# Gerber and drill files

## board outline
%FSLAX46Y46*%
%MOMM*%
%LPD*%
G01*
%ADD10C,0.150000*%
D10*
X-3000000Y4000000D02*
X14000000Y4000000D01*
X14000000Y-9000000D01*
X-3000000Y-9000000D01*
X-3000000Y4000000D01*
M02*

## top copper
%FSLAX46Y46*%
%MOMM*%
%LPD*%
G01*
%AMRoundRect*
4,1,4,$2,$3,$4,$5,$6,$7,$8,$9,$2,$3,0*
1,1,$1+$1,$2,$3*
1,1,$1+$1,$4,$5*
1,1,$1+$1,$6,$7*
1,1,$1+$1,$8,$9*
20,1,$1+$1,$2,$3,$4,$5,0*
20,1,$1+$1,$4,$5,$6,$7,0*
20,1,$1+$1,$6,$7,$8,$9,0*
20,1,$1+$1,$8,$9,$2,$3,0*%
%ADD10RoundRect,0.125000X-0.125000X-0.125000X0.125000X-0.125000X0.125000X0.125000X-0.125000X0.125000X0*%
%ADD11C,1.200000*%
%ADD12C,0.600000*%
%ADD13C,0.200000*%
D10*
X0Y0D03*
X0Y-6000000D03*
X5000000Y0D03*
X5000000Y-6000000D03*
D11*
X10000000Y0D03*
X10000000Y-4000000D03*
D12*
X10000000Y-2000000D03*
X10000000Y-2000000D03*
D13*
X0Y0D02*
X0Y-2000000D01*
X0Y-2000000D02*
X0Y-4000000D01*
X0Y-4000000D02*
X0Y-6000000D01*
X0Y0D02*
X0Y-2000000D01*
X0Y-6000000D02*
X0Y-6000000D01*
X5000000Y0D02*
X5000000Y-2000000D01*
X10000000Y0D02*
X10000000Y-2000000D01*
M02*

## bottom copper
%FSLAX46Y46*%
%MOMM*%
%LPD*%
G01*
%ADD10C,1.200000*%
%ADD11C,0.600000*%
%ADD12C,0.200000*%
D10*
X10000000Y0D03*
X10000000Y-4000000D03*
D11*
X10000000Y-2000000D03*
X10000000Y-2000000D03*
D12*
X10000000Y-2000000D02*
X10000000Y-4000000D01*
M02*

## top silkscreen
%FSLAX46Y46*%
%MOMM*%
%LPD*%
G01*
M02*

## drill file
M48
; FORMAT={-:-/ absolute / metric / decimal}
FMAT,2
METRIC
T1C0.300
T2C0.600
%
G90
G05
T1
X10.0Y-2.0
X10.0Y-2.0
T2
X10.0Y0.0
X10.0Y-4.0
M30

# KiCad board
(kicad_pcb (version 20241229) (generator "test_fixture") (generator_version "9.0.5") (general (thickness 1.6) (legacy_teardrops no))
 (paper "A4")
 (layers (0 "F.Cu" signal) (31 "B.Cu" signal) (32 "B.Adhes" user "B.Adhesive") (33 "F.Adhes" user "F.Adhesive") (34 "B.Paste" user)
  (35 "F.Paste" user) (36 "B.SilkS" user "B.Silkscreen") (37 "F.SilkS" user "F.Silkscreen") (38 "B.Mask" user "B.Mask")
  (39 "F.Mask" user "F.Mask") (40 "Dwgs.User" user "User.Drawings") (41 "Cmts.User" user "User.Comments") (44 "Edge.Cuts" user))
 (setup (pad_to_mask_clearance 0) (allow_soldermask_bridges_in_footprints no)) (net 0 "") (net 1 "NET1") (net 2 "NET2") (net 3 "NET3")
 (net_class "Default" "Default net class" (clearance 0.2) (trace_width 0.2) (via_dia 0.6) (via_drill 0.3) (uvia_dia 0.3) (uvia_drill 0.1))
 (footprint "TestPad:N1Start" (layer "F.Cu") (at 0 0)
  (pad "1" smd roundrect (at 0 0) (size 0.5 0.5) (layers "F.Cu" "F.Paste" "F.Mask") (roundrect_rratio 0.25) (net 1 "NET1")))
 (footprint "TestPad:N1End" (layer "F.Cu") (at 0 6)
  (pad "1" smd roundrect (at 0 0) (size 0.5 0.5) (layers "F.Cu" "F.Paste" "F.Mask") (roundrect_rratio 0.25) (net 1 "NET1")))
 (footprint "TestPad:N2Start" (layer "F.Cu") (at 5 0)
  (pad "1" smd roundrect (at 0 0) (size 0.5 0.5) (layers "F.Cu" "F.Paste" "F.Mask") (roundrect_rratio 0.25) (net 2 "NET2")))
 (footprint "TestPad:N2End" (layer "F.Cu") (at 5 6)
  (pad "1" smd roundrect (at 0 0) (size 0.5 0.5) (layers "F.Cu" "F.Paste" "F.Mask") (roundrect_rratio 0.25) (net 2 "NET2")))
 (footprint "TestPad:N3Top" (layer "F.Cu") (at 10 0)
  (pad "1" thru_hole circle (at 0 0) (size 1.2 1.2) (drill 0.6) (layers "*.Cu" "*.Mask") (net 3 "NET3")))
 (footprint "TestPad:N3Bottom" (layer "F.Cu") (at 10 4)
  (pad "1" thru_hole circle (at 0 0) (size 1.2 1.2) (drill 0.6) (layers "*.Cu" "*.Mask") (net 3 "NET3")))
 (segment (start 0 0) (end 0 2) (width 0.2) (layer "F.Cu") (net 1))
 (segment (start 0 2) (end 0 4) (width 0.2) (layer "F.Cu") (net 1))
 (segment (start 0 4) (end 0 6) (width 0.2) (layer "F.Cu") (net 1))
 (segment (start 0 0) (end 0 2) (width 0.2) (layer "F.Cu") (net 1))
 (segment (start 0 6) (end 0 6) (width 0.2) (layer "F.Cu") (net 1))
 (segment (start 5 0) (end 5 2) (width 0.2) (layer "F.Cu") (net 2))
 (segment (start 10 0) (end 10 2) (width 0.2) (layer "F.Cu") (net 3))
 (segment (start 10 2) (end 10 4) (width 0.2) (layer "B.Cu") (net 3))
 (via (at 10 2) (size 0.6) (drill 0.3) (layers "F.Cu" "B.Cu") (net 3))
 (via (at 10 2) (size 0.6) (drill 0.3) (layers "F.Cu" "B.Cu") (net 3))
 (gr_rect (start -3 -4) (end 14 9) (stroke (width 0.15) (type solid)) (fill none) (layer "Edge.Cuts")))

